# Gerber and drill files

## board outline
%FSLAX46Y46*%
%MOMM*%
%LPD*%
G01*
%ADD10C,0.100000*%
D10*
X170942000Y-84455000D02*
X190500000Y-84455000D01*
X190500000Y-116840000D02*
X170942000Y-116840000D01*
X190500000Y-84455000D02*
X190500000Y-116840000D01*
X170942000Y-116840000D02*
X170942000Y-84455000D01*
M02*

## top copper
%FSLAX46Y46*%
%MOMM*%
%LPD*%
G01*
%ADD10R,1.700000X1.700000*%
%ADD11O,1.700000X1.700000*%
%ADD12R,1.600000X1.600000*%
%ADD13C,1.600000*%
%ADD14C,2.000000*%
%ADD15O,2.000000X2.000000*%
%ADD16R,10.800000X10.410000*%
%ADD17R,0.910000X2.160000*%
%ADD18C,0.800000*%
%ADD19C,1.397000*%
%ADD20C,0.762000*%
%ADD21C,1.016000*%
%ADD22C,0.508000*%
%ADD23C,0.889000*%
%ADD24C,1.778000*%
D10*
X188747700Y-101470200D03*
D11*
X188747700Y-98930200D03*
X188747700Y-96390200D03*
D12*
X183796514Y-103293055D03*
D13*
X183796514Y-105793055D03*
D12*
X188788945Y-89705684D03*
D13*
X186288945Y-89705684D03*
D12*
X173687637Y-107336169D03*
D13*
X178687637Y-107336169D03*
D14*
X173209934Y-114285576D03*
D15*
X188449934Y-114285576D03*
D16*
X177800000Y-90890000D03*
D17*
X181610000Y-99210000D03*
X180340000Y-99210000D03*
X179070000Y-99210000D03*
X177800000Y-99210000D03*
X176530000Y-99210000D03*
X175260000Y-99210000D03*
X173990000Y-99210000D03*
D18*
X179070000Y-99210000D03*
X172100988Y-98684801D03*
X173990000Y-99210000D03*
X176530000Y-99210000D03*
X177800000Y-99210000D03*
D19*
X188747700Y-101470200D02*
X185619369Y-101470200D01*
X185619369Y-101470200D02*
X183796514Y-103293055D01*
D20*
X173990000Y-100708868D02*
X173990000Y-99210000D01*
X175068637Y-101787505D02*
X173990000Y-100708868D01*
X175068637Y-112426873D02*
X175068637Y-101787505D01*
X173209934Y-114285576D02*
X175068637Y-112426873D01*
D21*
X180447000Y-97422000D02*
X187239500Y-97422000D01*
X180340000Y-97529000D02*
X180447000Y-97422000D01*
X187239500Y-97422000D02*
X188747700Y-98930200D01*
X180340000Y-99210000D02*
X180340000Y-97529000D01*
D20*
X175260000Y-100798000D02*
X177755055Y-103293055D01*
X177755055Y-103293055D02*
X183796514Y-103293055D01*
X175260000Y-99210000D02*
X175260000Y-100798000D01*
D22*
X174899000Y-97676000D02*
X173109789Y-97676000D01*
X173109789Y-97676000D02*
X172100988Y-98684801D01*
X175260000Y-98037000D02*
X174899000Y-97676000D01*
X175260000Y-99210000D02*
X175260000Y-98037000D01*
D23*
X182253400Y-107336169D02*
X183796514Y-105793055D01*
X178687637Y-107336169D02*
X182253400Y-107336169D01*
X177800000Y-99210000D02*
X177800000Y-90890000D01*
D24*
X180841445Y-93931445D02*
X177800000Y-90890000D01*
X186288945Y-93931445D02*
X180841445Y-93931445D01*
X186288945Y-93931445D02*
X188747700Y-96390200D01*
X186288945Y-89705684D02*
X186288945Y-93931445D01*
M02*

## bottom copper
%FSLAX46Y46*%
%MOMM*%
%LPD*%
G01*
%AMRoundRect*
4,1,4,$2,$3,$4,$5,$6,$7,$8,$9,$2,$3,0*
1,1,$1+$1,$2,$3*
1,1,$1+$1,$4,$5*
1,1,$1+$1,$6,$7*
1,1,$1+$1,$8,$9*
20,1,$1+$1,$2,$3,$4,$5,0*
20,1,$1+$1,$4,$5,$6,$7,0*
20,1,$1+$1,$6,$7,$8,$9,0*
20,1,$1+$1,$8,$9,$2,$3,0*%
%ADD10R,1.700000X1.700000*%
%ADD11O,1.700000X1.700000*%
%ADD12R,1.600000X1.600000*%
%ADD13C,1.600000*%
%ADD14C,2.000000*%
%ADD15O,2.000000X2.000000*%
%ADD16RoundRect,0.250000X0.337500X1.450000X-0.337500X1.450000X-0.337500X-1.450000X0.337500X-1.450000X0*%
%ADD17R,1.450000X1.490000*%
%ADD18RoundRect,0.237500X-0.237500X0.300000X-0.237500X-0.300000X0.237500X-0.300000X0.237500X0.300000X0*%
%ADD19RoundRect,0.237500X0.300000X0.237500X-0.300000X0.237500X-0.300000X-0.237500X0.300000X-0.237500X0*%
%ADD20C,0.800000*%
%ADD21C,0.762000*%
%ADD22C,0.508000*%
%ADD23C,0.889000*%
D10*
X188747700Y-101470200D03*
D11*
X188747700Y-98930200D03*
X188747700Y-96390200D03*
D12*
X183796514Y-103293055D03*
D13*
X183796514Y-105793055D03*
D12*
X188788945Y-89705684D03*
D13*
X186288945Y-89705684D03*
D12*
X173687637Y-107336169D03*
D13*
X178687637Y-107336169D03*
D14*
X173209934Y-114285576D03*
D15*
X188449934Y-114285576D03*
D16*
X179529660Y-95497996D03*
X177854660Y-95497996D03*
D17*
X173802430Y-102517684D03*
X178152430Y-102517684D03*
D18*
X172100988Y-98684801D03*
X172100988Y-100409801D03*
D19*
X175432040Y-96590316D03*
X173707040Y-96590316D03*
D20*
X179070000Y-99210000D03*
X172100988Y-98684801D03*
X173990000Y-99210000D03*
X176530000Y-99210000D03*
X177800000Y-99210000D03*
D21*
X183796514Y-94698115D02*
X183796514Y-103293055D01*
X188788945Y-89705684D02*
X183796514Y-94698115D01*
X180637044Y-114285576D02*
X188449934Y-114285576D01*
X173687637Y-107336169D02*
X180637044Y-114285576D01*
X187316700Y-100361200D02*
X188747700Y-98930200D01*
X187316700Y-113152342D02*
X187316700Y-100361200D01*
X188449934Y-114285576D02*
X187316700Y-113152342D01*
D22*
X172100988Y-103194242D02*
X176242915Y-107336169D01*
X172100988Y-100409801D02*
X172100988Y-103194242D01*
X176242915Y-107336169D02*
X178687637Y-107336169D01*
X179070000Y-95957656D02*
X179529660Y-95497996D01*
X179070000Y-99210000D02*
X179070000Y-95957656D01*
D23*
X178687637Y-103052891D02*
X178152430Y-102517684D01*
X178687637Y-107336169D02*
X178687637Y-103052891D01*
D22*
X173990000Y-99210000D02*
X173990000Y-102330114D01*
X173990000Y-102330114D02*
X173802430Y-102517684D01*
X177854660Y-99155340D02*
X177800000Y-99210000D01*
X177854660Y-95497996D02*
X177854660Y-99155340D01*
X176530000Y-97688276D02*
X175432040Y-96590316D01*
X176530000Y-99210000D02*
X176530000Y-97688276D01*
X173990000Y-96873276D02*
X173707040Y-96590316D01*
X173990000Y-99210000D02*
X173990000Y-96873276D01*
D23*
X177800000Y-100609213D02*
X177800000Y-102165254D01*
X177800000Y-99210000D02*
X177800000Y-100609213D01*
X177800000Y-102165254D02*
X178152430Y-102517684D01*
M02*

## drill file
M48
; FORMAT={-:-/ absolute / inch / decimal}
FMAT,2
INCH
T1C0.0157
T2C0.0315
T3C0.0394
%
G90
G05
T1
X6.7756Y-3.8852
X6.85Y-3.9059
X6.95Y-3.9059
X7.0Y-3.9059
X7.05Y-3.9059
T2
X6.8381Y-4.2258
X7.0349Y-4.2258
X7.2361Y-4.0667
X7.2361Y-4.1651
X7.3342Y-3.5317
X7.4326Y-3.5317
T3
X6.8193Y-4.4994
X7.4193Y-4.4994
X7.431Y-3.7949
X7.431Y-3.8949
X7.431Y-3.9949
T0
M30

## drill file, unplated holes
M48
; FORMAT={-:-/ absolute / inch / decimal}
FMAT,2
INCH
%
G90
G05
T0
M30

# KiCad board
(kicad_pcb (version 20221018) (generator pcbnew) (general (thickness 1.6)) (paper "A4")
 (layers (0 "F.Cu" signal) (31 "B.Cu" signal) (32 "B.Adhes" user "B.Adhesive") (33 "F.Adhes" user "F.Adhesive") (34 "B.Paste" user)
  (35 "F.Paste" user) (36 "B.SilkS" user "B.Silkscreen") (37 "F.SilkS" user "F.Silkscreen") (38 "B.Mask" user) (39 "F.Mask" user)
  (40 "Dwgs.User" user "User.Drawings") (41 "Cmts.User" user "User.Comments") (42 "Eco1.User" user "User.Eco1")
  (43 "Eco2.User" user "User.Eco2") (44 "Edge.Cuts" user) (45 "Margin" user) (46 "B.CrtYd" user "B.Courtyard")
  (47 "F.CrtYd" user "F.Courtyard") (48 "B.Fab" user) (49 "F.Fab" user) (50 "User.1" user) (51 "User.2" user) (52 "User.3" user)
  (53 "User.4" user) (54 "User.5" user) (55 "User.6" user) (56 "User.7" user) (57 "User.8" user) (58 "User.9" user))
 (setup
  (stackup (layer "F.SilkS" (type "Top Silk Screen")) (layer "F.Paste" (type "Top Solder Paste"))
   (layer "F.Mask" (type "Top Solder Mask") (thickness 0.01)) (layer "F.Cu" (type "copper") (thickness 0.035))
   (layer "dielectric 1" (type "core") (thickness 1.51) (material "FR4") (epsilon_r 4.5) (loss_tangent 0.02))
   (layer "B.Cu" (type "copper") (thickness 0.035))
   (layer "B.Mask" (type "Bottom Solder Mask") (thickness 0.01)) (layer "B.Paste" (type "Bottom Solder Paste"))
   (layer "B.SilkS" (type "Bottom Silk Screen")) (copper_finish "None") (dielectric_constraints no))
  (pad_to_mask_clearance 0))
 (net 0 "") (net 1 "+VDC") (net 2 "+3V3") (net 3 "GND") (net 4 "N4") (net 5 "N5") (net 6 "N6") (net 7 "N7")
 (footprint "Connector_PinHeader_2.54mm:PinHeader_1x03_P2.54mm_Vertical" (layer "F.Cu") (at 188.7477 101.4702 180)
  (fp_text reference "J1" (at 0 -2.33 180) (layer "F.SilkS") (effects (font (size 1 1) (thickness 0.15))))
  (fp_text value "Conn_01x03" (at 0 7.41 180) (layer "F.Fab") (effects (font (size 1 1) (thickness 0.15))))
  (pad "1" thru_hole rect (at 0 0 180) (size 1.7 1.7) (drill 1) (layers "*.Cu" "*.Mask") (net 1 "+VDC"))
  (pad "2" thru_hole oval (at 0 2.54 180) (size 1.7 1.7) (drill 1) (layers "*.Cu" "*.Mask") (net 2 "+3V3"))
  (pad "3" thru_hole oval (at 0 5.08 180) (size 1.7 1.7) (drill 1) (layers "*.Cu" "*.Mask") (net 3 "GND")))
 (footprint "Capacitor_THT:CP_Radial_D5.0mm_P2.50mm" (layer "F.Cu") (at 183.796514 103.293055 -90)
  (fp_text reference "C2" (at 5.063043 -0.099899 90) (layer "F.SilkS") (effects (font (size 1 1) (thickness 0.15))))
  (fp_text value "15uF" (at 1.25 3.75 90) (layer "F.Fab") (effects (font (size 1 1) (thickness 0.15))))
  (pad "1" thru_hole rect (at 0 0 270) (size 1.6 1.6) (drill 0.8) (layers "*.Cu" "*.Mask") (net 1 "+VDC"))
  (pad "2" thru_hole circle (at 2.5 0 270) (size 1.6 1.6) (drill 0.8) (layers "*.Cu" "*.Mask") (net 3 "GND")))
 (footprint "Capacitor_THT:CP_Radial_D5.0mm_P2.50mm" (layer "F.Cu") (at 188.788945 89.705684 180)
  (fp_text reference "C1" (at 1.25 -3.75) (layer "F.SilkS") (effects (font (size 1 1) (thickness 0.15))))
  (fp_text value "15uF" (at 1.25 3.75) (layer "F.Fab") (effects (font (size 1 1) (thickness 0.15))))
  (pad "1" thru_hole rect (at 0 0 180) (size 1.6 1.6) (drill 0.8) (layers "*.Cu" "*.Mask") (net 1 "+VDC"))
  (pad "2" thru_hole circle (at 2.5 0 180) (size 1.6 1.6) (drill 0.8) (layers "*.Cu" "*.Mask") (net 3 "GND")))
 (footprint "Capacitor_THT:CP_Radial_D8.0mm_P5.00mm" (layer "F.Cu") (at 173.687637 107.336169)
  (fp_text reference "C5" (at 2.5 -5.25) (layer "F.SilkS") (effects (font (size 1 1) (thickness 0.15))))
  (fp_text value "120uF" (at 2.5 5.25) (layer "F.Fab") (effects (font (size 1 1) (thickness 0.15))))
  (pad "1" thru_hole rect (at 0 0) (size 1.6 1.6) (drill 0.8) (layers "*.Cu" "*.Mask") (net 2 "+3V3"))
  (pad "2" thru_hole circle (at 5 0) (size 1.6 1.6) (drill 0.8) (layers "*.Cu" "*.Mask") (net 3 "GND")))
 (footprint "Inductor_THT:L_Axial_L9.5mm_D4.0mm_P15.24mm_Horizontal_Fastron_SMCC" (layer "F.Cu") (at 173.209934 114.285576)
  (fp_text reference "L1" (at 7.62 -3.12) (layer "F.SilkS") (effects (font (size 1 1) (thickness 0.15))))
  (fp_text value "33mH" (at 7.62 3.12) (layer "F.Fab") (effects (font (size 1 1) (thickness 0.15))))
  (pad "1" thru_hole circle (at 0 0) (size 2 2) (drill 1) (layers "*.Cu" "*.Mask") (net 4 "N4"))
  (pad "2" thru_hole oval (at 15.24 0) (size 2 2) (drill 1) (layers "*.Cu" "*.Mask") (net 2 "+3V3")))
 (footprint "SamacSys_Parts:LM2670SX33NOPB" (layer "F.Cu") (at 177.8 91.44 -90)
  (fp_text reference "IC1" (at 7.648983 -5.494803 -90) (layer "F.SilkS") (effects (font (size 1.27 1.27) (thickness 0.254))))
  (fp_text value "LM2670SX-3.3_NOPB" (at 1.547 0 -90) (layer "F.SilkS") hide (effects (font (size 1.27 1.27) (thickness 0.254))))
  (pad "1" smd rect (at 7.77 3.81) (size 0.91 2.16) (layers "F.Cu" "F.Paste" "F.Mask") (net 4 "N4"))
  (pad "2" smd rect (at 7.77 2.54) (size 0.91 2.16) (layers "F.Cu" "F.Paste" "F.Mask") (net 1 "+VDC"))
  (pad "3" smd rect (at 7.77 1.27) (size 0.91 2.16) (layers "F.Cu" "F.Paste" "F.Mask") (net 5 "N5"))
  (pad "4" smd rect (at 7.77 0) (size 0.91 2.16) (layers "F.Cu" "F.Paste" "F.Mask") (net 3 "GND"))
  (pad "5" smd rect (at 7.77 -1.27) (size 0.91 2.16) (layers "F.Cu" "F.Paste" "F.Mask") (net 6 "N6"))
  (pad "6" smd rect (at 7.77 -2.54) (size 0.91 2.16) (layers "F.Cu" "F.Paste" "F.Mask") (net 2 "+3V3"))
  (pad "7" smd rect (at 7.77 -3.81) (size 0.91 2.16) (layers "F.Cu" "F.Paste" "F.Mask") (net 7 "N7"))
  (pad "8" smd rect (at -0.55 0 270) (size 10.41 10.8) (layers "F.Cu" "F.Paste" "F.Mask") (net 3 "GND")))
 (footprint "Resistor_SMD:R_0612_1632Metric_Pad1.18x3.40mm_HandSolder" (layer "B.Cu") (at 178.69216 95.497996 180)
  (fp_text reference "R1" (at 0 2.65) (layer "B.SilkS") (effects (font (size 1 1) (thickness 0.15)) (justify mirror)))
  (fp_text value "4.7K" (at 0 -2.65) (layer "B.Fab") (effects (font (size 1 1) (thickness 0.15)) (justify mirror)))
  (pad "1" smd roundrect (at -0.8375 0 180) (size 1.175 3.4) (layers "B.Cu" "B.Paste" "B.Mask") (roundrect_rratio 0.2127659574) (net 6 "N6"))
  (pad "2" smd roundrect (at 0.8375 0 180) (size 1.175 3.4) (layers "B.Cu" "B.Paste" "B.Mask") (roundrect_rratio 0.2127659574) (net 3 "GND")))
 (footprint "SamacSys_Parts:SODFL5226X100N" (layer "B.Cu") (at 175.97743 102.517684)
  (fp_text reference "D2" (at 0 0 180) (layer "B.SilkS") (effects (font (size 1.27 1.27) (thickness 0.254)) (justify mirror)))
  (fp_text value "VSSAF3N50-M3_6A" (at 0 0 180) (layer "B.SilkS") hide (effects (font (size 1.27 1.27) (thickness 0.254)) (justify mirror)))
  (pad "1" smd rect (at -2.175 0) (size 1.45 1.49) (layers "B.Cu" "B.Paste" "B.Mask") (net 4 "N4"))
  (pad "2" smd rect (at 2.175 0) (size 1.45 1.49) (layers "B.Cu" "B.Paste" "B.Mask") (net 3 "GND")))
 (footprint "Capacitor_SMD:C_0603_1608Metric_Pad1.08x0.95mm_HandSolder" (layer "B.Cu") (at 172.100988 99.547301 -90)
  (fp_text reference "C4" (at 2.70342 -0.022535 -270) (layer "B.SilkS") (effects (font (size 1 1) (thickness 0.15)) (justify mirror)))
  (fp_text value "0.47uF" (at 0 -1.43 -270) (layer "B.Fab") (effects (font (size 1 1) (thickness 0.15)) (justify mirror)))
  (pad "1" smd roundrect (at -0.8625 0 270) (size 1.075 0.95) (layers "B.Cu" "B.Paste" "B.Mask") (roundrect_rratio 0.25) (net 1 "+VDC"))
  (pad "2" smd roundrect (at 0.8625 0 270) (size 1.075 0.95) (layers "B.Cu" "B.Paste" "B.Mask") (roundrect_rratio 0.25) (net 3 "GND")))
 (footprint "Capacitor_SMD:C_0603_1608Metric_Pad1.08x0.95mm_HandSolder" (layer "B.Cu") (at 174.56954 96.590316 180)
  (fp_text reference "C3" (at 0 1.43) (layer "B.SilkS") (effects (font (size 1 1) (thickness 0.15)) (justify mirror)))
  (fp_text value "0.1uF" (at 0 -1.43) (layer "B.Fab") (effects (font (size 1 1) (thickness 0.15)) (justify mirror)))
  (pad "1" smd roundrect (at -0.8625 0 180) (size 1.075 0.95) (layers "B.Cu" "B.Paste" "B.Mask") (roundrect_rratio 0.25) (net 5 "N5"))
  (pad "2" smd roundrect (at 0.8625 0 180) (size 1.075 0.95) (layers "B.Cu" "B.Paste" "B.Mask") (roundrect_rratio 0.25) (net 4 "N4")))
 (gr_line (start 170.942 84.455) (end 190.5 84.455) (stroke (width 0.1) (type solid)) (layer "Edge.Cuts"))
 (gr_line (start 190.5 116.84) (end 170.942 116.84) (stroke (width 0.1) (type default)) (layer "Edge.Cuts"))
 (gr_line (start 190.5 84.455) (end 190.5 116.84) (stroke (width 0.1) (type default)) (layer "Edge.Cuts"))
 (gr_line (start 170.942 116.84) (end 170.942 84.455) (stroke (width 0.1) (type solid)) (layer "Edge.Cuts"))
 (segment (start 175.26 100.798) (end 177.755055 103.293055) (width 0.762) (layer "F.Cu") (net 1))
 (segment (start 185.619369 101.4702) (end 183.796514 103.293055) (width 1.397) (layer "F.Cu") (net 1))
 (segment (start 174.899 97.676) (end 173.109789 97.676) (width 0.508) (layer "F.Cu") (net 1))
 (segment (start 188.7477 101.4702) (end 185.619369 101.4702) (width 1.397) (layer "F.Cu") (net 1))
 (segment (start 175.26 99.21) (end 175.26 100.798) (width 0.762) (layer "F.Cu") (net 1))
 (segment (start 177.755055 103.293055) (end 183.796514 103.293055) (width 0.762) (layer "F.Cu") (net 1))
 (segment (start 175.26 99.21) (end 175.26 98.037) (width 0.508) (layer "F.Cu") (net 1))
 (segment (start 175.26 98.037) (end 174.899 97.676) (width 0.508) (layer "F.Cu") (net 1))
 (segment (start 173.109789 97.676) (end 172.100988 98.684801) (width 0.508) (layer "F.Cu") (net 1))
 (via (at 172.100988 98.684801) (size 0.8) (drill 0.4) (layers "F.Cu" "B.Cu") (free) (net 1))
 (segment (start 183.796514 94.698115) (end 183.796514 103.293055) (width 0.762) (layer "B.Cu") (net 1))
 (segment (start 188.788945 89.705684) (end 183.796514 94.698115) (width 0.762) (layer "B.Cu") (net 1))
 (segment (start 186.288945 89.705684) (end 186.288945 93.931445) (width 1.778) (layer "F.Cu") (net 3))
 (segment (start 177.8 99.21) (end 177.8 90.89) (width 0.889) (layer "F.Cu") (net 3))
 (segment (start 178.687637 107.336169) (end 182.2534 107.336169) (width 0.889) (layer "F.Cu") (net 3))
 (segment (start 182.2534 107.336169) (end 183.796514 105.793055) (width 0.889) (layer "F.Cu") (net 3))
 (segment (start 180.841445 93.931445) (end 177.8 90.89) (width 1.778) (layer "F.Cu") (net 3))
 (segment (start 186.288945 93.931445) (end 180.841445 93.931445) (width 1.778) (layer "F.Cu") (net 3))
 (segment (start 186.288945 93.931445) (end 188.7477 96.3902) (width 1.778) (layer "F.Cu") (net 3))
 (via (at 177.8 99.21) (size 0.8) (drill 0.4) (layers "F.Cu" "B.Cu") (free) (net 3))
 (segment (start 172.100988 100.409801) (end 172.100988 103.194242) (width 0.508) (layer "B.Cu") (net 3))
 (segment (start 177.85466 95.497996) (end 177.85466 99.15534) (width 0.508) (layer "B.Cu") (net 3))
 (segment (start 177.8 102.165254) (end 178.15243 102.517684) (width 0.889) (layer "B.Cu") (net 3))
 (segment (start 177.85466 99.15534) (end 177.8 99.21) (width 0.508) (layer "B.Cu") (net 3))
 (segment (start 177.8 99.21) (end 177.8 100.609213) (width 0.889) (layer "B.Cu") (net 3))
 (segment (start 176.242915 107.336169) (end 178.687637 107.336169) (width 0.508) (layer "B.Cu") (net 3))
 (segment (start 178.687637 107.336169) (end 178.687637 103.052891) (width 0.889) (layer "B.Cu") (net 3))
 (segment (start 177.8 100.609213) (end 177.8 102.165254) (width 0.889) (layer "B.Cu") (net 3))
 (segment (start 178.687637 103.052891) (end 178.15243 102.517684) (width 0.889) (layer "B.Cu") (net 3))
 (segment (start 172.100988 103.194242) (end 176.242915 107.336169) (width 0.508) (layer "B.Cu") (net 3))
 (via (at 176.53 99.21) (size 0.8) (drill 0.4) (layers "F.Cu" "B.Cu") (free) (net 5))
 (segment (start 176.53 97.688276) (end 175.43204 96.590316) (width 0.508) (layer "B.Cu") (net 5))
 (segment (start 176.53 99.21) (end 176.53 97.688276) (width 0.508) (layer "B.Cu") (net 5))
 (segment (start 175.068637 101.787505) (end 173.99 100.708868) (width 0.762) (layer "F.Cu") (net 4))
 (segment (start 173.209934 114.285576) (end 175.068637 112.426873) (width 0.762) (layer "F.Cu") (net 4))
 (segment (start 173.99 100.708868) (end 173.99 99.21) (width 0.762) (layer "F.Cu") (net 4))
 (segment (start 175.068637 112.426873) (end 175.068637 101.787505) (width 0.762) (layer "F.Cu") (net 4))
 (via (at 173.99 99.21) (size 0.8) (drill 0.4) (layers "F.Cu" "B.Cu") (free) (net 4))
 (segment (start 173.99 102.330114) (end 173.80243 102.517684) (width 0.508) (layer "B.Cu") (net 4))
 (segment (start 173.99 96.873276) (end 173.70704 96.590316) (width 0.508) (layer "B.Cu") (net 4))
 (segment (start 173.99 99.21) (end 173.99 102.330114) (width 0.508) (layer "B.Cu") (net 4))
 (segment (start 173.99 99.21) (end 173.99 96.873276) (width 0.508) (layer "B.Cu") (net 4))
 (segment (start 180.34 97.529) (end 180.447 97.422) (width 1.016) (layer "F.Cu") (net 2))
 (segment (start 180.34 99.21) (end 180.34 97.529) (width 1.016) (layer "F.Cu") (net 2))
 (segment (start 180.447 97.422) (end 187.2395 97.422) (width 1.016) (layer "F.Cu") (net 2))
 (segment (start 187.2395 97.422) (end 188.7477 98.9302) (width 1.016) (layer "F.Cu") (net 2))
 (segment (start 173.687637 107.336169) (end 180.637044 114.285576) (width 0.762) (layer "B.Cu") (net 2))
 (segment (start 188.449934 114.285576) (end 187.3167 113.152342) (width 0.762) (layer "B.Cu") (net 2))
 (segment (start 180.637044 114.285576) (end 188.449934 114.285576) (width 0.762) (layer "B.Cu") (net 2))
 (segment (start 187.3167 113.152342) (end 187.3167 100.3612) (width 0.762) (layer "B.Cu") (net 2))
 (segment (start 187.3167 100.3612) (end 188.7477 98.9302) (width 0.762) (layer "B.Cu") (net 2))
 (via (at 179.07 99.21) (size 0.8) (drill 0.4) (layers "F.Cu" "B.Cu") (free) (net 6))
 (segment (start 179.07 99.21) (end 179.07 95.957656) (width 0.508) (layer "B.Cu") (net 6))
 (segment (start 179.07 95.957656) (end 179.52966 95.497996) (width 0.508) (layer "B.Cu") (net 6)))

